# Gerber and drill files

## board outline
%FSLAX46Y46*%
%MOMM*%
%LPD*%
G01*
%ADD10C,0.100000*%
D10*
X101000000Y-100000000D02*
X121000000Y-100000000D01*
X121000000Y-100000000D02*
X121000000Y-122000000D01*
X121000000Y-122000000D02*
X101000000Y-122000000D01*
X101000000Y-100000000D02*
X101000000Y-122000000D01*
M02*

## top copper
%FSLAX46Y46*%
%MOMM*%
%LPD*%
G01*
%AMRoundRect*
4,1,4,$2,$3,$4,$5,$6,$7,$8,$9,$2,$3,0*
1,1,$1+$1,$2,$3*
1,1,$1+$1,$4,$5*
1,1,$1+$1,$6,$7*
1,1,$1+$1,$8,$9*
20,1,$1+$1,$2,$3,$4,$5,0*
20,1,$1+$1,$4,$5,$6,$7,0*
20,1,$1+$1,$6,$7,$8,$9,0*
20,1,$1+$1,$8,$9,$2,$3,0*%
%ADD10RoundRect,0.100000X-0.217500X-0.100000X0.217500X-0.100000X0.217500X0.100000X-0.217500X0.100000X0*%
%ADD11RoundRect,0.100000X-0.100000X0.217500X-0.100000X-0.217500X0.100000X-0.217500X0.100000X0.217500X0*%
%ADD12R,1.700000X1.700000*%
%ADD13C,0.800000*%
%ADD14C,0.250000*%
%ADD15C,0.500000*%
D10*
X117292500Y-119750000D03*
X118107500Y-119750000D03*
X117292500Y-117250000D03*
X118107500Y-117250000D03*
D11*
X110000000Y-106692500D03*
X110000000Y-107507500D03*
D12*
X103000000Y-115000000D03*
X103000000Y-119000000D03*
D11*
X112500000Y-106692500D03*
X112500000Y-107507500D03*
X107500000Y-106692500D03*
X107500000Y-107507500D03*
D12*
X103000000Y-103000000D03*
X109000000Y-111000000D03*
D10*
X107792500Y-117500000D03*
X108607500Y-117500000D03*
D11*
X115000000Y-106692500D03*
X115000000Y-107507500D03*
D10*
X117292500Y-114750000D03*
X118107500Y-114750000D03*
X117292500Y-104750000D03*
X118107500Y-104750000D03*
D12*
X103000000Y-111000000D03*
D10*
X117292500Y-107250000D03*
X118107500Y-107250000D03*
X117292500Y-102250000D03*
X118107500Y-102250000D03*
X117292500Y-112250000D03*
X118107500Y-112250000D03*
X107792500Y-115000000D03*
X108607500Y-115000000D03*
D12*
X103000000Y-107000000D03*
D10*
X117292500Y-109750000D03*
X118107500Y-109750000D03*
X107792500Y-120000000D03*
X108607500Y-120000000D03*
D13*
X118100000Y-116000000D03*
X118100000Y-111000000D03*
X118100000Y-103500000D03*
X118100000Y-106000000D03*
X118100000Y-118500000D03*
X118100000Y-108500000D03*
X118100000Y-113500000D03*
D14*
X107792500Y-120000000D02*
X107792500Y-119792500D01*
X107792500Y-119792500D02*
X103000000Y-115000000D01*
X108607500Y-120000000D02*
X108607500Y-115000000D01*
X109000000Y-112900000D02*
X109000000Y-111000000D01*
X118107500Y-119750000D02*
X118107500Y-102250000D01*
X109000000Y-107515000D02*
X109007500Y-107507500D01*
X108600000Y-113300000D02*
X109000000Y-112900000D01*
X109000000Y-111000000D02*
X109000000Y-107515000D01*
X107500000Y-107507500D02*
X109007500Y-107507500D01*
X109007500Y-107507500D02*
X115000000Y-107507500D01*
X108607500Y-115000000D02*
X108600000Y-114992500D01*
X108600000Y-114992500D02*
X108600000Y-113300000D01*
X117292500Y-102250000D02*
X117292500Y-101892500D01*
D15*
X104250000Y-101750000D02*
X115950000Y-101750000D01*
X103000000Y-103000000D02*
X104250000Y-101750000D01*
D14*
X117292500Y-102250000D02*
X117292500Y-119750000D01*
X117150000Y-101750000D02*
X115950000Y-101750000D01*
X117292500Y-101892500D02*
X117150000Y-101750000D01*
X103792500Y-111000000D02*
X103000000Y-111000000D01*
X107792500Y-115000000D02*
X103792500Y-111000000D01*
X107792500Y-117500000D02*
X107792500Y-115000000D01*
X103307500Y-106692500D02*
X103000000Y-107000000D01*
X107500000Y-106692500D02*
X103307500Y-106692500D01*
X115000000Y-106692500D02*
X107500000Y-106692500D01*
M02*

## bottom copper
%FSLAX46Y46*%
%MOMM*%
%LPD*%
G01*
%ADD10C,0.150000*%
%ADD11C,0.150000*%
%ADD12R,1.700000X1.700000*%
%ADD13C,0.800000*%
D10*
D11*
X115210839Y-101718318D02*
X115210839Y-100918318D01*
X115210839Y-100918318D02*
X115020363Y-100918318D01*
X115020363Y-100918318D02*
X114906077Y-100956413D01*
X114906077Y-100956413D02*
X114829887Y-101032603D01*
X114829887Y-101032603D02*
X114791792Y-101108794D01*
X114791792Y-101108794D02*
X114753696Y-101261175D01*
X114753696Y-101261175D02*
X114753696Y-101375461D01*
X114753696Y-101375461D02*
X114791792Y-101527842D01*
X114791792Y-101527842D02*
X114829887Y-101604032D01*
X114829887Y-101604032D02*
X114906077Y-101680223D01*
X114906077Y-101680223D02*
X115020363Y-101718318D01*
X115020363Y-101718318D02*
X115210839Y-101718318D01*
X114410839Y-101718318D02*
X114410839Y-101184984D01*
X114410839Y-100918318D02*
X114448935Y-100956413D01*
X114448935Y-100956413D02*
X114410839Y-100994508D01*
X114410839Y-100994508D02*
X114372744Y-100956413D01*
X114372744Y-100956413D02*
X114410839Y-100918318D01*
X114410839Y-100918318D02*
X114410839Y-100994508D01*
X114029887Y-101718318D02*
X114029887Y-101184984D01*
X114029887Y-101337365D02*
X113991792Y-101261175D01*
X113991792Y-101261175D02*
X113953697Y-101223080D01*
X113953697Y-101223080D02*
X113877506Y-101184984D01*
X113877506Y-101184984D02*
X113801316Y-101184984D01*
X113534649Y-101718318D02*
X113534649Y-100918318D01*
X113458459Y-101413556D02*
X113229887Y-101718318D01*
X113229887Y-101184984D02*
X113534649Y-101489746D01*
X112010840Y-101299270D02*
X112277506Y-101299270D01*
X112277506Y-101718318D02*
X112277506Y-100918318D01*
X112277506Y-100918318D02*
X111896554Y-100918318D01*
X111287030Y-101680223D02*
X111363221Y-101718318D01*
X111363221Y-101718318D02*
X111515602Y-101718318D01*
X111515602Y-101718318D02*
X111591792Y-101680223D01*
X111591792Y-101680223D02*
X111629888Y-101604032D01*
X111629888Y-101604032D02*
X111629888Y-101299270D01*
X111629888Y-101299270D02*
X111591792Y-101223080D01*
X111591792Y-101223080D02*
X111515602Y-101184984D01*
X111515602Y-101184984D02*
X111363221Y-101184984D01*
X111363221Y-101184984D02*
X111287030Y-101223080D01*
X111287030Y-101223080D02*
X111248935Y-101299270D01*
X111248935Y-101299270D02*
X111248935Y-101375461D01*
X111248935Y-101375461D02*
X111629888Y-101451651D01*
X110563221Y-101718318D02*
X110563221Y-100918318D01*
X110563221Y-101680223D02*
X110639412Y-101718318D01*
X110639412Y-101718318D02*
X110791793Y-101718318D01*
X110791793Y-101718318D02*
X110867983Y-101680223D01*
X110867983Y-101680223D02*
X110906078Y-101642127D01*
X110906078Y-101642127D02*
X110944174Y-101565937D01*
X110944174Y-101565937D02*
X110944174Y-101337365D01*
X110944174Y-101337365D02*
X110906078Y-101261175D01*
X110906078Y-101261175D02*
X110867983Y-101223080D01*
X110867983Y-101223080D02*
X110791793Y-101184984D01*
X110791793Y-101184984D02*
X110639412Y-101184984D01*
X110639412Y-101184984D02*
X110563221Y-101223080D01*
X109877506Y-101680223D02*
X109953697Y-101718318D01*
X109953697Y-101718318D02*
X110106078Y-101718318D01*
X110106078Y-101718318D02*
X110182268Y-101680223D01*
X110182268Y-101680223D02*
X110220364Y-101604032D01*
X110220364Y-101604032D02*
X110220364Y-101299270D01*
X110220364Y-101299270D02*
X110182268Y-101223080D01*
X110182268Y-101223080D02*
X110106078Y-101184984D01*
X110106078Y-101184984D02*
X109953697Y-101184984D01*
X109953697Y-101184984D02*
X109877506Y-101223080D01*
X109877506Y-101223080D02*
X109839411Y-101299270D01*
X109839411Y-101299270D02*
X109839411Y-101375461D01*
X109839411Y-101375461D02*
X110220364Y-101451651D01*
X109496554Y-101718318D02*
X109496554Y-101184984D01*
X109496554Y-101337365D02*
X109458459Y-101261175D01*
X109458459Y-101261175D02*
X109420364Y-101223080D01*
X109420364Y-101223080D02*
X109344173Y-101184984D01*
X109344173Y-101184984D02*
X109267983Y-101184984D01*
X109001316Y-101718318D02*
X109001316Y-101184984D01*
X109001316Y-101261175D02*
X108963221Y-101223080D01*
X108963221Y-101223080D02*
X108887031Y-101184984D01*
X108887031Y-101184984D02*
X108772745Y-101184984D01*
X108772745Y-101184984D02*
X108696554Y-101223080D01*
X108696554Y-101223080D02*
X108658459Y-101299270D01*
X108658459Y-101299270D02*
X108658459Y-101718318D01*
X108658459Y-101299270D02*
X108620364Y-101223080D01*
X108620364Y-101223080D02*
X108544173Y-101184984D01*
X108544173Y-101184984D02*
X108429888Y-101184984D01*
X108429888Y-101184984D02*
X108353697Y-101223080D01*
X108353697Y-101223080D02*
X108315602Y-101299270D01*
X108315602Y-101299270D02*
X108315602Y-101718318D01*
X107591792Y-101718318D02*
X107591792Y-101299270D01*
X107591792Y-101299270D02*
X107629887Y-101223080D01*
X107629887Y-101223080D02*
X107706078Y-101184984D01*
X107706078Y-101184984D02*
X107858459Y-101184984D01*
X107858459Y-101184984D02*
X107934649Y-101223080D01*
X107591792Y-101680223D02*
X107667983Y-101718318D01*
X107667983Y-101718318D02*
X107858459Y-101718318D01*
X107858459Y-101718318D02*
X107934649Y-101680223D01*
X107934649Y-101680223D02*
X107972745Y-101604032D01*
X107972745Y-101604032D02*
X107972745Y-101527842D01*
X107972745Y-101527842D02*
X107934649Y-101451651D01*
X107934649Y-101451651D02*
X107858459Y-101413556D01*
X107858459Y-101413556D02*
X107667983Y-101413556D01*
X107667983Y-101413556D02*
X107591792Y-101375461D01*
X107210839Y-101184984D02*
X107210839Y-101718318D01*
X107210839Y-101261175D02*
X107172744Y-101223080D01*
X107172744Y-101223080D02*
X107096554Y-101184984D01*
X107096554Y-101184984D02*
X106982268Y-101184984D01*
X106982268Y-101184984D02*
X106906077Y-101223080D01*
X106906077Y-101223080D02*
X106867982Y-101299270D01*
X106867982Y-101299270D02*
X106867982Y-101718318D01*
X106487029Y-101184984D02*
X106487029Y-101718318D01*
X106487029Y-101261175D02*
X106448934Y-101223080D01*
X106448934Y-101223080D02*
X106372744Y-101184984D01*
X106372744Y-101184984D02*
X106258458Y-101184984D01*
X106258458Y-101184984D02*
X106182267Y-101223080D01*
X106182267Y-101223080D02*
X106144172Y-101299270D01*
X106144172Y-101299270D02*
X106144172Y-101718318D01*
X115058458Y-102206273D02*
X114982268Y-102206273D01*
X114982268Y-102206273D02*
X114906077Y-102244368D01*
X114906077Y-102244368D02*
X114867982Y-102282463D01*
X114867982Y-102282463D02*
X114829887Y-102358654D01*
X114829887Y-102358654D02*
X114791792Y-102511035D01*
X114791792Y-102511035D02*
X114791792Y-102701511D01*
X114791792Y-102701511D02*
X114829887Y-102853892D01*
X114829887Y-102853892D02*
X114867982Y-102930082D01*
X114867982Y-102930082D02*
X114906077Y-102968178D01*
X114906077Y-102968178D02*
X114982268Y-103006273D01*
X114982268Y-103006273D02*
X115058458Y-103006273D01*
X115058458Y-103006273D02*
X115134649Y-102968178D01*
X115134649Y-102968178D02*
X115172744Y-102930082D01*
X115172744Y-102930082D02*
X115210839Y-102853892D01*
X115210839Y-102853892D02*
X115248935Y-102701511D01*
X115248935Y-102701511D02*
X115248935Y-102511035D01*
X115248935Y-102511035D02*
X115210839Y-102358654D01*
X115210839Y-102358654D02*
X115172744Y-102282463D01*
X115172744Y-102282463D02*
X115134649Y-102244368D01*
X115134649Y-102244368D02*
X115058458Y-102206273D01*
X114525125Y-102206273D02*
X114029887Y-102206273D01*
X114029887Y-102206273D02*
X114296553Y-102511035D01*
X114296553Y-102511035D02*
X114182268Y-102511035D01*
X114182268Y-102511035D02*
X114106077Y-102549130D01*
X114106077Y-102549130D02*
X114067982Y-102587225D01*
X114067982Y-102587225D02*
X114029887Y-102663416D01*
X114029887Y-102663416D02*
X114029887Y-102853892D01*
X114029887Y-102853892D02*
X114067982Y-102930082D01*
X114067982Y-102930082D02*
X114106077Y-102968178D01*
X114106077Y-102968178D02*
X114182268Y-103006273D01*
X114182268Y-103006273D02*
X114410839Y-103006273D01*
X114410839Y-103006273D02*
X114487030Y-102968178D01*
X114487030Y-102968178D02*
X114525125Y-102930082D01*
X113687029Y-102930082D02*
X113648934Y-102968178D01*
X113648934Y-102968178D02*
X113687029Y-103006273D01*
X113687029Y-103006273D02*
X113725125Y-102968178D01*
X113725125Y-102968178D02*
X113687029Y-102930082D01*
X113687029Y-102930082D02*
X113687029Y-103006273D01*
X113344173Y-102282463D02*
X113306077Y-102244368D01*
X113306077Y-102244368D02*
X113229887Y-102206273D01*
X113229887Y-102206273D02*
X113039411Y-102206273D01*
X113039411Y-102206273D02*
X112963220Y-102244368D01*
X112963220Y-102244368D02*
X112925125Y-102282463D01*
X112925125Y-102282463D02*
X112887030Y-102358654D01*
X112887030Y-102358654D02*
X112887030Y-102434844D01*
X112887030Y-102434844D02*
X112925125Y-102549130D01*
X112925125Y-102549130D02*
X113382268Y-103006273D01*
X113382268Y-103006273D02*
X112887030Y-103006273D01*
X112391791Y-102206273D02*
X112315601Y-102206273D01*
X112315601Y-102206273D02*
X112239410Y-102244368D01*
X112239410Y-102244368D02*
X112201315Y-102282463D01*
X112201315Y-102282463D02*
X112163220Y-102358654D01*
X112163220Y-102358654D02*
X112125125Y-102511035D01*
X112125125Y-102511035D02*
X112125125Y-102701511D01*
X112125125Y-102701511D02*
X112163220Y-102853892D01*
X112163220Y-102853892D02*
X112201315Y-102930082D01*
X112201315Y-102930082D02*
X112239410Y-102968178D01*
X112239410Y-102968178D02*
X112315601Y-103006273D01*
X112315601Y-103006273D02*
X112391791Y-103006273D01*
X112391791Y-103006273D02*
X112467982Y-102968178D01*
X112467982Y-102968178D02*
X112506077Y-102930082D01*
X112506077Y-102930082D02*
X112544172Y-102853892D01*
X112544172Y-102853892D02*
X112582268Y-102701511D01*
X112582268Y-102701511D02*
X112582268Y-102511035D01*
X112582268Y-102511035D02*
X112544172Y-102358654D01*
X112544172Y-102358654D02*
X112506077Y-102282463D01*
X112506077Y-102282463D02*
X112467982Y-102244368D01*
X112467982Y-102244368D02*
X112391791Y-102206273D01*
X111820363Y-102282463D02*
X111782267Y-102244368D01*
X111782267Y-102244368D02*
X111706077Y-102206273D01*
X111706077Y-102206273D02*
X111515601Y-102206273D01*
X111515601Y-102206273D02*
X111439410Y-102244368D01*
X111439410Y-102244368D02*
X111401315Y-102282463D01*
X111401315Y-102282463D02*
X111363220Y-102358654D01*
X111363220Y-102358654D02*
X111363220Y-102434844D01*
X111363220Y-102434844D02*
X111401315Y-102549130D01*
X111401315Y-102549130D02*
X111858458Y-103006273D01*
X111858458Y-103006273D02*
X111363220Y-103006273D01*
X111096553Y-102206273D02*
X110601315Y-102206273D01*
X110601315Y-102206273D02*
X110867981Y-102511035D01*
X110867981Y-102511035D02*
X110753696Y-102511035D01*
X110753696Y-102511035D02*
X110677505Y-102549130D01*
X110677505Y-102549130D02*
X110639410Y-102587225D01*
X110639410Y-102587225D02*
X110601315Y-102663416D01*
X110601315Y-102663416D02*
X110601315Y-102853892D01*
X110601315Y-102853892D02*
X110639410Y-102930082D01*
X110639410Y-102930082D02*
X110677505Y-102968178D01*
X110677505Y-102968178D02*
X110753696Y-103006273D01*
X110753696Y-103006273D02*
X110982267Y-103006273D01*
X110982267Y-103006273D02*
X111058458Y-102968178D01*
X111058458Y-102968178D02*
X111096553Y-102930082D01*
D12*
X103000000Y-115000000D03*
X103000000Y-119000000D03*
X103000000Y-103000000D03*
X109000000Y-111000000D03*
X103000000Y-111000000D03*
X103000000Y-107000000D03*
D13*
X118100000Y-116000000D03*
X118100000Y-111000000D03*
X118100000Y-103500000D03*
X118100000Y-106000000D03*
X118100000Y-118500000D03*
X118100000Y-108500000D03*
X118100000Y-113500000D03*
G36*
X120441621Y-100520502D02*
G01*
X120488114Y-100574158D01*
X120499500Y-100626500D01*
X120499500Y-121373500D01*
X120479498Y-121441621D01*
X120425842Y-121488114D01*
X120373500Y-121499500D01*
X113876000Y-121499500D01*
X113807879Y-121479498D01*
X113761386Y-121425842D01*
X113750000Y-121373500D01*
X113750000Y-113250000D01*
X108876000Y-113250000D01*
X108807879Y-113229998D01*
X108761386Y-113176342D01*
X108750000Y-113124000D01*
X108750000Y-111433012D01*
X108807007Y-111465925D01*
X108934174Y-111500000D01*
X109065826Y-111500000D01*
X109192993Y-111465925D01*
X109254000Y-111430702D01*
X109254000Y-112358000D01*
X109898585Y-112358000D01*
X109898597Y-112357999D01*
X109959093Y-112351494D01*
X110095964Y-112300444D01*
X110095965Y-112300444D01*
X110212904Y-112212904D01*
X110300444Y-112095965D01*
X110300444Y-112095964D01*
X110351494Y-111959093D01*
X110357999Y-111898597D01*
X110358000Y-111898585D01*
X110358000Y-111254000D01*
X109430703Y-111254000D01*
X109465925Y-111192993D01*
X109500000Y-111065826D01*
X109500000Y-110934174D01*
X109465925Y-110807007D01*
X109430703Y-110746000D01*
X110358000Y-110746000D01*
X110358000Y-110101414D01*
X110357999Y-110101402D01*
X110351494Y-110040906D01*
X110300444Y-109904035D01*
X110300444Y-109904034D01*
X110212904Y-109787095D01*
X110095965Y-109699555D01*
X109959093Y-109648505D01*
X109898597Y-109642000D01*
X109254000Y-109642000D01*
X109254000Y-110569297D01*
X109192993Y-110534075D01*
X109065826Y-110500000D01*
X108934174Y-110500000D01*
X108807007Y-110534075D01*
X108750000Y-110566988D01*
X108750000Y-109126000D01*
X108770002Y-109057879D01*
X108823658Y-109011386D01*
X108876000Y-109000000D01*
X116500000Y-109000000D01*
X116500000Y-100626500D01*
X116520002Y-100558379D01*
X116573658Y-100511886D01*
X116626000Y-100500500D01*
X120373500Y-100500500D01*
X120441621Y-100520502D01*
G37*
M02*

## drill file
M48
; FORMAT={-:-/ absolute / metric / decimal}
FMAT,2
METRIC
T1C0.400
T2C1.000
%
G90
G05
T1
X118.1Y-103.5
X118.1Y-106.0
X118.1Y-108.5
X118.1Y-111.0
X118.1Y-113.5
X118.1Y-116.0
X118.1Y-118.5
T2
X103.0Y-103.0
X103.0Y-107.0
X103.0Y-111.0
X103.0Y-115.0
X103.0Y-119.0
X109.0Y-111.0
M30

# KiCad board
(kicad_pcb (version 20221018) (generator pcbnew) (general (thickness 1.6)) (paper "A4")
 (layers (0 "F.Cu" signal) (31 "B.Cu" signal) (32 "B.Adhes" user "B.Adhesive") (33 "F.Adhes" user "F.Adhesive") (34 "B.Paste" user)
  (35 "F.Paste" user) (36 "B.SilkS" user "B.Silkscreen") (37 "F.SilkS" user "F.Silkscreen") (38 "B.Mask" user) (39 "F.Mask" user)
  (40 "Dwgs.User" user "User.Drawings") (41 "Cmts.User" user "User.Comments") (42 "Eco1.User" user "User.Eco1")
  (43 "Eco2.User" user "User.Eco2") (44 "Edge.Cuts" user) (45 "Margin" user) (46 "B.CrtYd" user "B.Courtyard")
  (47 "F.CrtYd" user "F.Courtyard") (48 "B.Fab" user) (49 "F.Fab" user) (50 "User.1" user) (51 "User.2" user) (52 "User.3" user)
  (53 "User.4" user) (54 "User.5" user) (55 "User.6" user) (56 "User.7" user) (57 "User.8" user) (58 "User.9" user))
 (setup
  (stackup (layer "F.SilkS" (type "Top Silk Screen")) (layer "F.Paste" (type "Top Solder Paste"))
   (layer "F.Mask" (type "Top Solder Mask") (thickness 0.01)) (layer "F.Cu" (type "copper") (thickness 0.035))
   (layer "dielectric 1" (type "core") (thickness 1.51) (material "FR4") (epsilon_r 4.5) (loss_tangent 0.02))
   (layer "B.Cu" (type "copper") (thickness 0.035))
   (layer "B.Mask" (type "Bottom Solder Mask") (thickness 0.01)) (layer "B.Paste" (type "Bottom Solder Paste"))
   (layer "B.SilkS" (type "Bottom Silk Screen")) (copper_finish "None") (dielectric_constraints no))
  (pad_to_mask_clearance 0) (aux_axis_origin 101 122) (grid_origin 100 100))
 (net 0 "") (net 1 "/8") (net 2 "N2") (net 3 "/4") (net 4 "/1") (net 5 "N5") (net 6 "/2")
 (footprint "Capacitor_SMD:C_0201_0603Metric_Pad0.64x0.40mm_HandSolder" (layer "F.Cu") (at 117.7 119.75)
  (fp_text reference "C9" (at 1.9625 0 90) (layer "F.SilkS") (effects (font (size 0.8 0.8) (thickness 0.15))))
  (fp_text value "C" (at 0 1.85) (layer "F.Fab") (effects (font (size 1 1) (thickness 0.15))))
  (pad "" smd roundrect (at -0.4325 0) (size 0.458 0.36) (layers "F.Paste") (roundrect_rratio 0.25))
  (pad "" smd roundrect (at 0.4325 0) (size 0.458 0.36) (layers "F.Paste") (roundrect_rratio 0.25))
  (pad "1" smd roundrect (at -0.4075 0) (size 0.635 0.4) (layers "F.Cu" "F.Mask") (roundrect_rratio 0.25) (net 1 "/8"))
  (pad "2" smd roundrect (at 0.4075 0) (size 0.635 0.4) (layers "F.Cu" "F.Mask") (roundrect_rratio 0.25) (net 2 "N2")))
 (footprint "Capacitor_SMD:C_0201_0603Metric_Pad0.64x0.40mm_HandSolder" (layer "F.Cu") (at 117.7 117.25)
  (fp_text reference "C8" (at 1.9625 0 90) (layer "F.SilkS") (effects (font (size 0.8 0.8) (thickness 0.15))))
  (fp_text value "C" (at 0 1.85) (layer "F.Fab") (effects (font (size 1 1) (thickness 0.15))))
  (pad "" smd roundrect (at -0.4325 0) (size 0.458 0.36) (layers "F.Paste") (roundrect_rratio 0.25))
  (pad "" smd roundrect (at 0.4325 0) (size 0.458 0.36) (layers "F.Paste") (roundrect_rratio 0.25))
  (pad "1" smd roundrect (at -0.4075 0) (size 0.635 0.4) (layers "F.Cu" "F.Mask") (roundrect_rratio 0.25) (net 1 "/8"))
  (pad "2" smd roundrect (at 0.4075 0) (size 0.635 0.4) (layers "F.Cu" "F.Mask") (roundrect_rratio 0.25) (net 2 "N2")))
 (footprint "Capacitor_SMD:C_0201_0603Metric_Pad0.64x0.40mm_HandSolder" (layer "F.Cu") (at 110 107.1 -90)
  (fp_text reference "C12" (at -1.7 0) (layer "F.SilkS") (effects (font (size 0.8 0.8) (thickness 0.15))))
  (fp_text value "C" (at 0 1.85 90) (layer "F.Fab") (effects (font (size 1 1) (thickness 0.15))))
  (pad "" smd roundrect (at -0.4325 0 270) (size 0.458 0.36) (layers "F.Paste") (roundrect_rratio 0.25))
  (pad "" smd roundrect (at 0.4325 0 270) (size 0.458 0.36) (layers "F.Paste") (roundrect_rratio 0.25))
  (pad "1" smd roundrect (at -0.4075 0 270) (size 0.635 0.4) (layers "F.Cu" "F.Mask") (roundrect_rratio 0.25) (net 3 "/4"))
  (pad "2" smd roundrect (at 0.4075 0 270) (size 0.635 0.4) (layers "F.Cu" "F.Mask") (roundrect_rratio 0.25) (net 2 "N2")))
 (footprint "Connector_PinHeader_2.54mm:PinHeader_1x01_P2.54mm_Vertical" (layer "F.Cu") (at 103 115)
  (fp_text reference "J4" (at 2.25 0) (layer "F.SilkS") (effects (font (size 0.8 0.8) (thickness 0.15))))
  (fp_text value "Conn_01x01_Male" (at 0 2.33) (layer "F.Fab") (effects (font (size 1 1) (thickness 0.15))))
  (pad "1" thru_hole rect (at 0 0) (size 1.7 1.7) (drill 1) (layers "*.Cu" "*.Mask") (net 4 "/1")))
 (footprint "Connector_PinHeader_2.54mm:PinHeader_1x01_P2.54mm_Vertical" (layer "F.Cu") (at 103 119)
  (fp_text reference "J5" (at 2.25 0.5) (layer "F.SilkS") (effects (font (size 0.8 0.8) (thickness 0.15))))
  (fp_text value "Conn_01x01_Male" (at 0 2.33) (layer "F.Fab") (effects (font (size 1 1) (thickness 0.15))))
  (pad "1" thru_hole rect (at 0 0) (size 1.7 1.7) (drill 1) (layers "*.Cu" "*.Mask") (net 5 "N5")))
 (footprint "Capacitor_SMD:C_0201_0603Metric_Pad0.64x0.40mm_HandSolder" (layer "F.Cu") (at 112.5 107.1 -90)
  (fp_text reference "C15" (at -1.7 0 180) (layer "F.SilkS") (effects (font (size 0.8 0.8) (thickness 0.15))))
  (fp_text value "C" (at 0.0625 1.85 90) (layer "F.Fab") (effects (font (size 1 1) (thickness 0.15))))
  (pad "" smd roundrect (at -0.4325 0 270) (size 0.458 0.36) (layers "F.Paste") (roundrect_rratio 0.25))
  (pad "" smd roundrect (at 0.4325 0 270) (size 0.458 0.36) (layers "F.Paste") (roundrect_rratio 0.25))
  (pad "1" smd roundrect (at -0.4075 0 270) (size 0.635 0.4) (layers "F.Cu" "F.Mask") (roundrect_rratio 0.25) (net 3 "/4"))
  (pad "2" smd roundrect (at 0.4075 0 270) (size 0.635 0.4) (layers "F.Cu" "F.Mask") (roundrect_rratio 0.25) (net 2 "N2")))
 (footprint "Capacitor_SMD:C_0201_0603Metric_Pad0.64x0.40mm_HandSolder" (layer "F.Cu") (at 107.5 107.1 -90)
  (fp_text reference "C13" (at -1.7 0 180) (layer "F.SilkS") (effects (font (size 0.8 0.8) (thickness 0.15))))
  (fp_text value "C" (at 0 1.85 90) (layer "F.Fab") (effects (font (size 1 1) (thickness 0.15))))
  (pad "" smd roundrect (at -0.4325 0 270) (size 0.458 0.36) (layers "F.Paste") (roundrect_rratio 0.25))
  (pad "" smd roundrect (at 0.4325 0 270) (size 0.458 0.36) (layers "F.Paste") (roundrect_rratio 0.25))
  (pad "1" smd roundrect (at -0.4075 0 270) (size 0.635 0.4) (layers "F.Cu" "F.Mask") (roundrect_rratio 0.25) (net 3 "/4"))
  (pad "2" smd roundrect (at 0.4075 0 270) (size 0.635 0.4) (layers "F.Cu" "F.Mask") (roundrect_rratio 0.25) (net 2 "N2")))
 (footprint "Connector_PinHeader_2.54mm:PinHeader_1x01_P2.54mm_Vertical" (layer "F.Cu") (at 103 103)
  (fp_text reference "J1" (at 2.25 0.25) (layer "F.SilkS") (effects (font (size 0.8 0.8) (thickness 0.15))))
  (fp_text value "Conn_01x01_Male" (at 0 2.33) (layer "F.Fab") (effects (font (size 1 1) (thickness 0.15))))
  (pad "1" thru_hole rect (at 0 0) (size 1.7 1.7) (drill 1) (layers "*.Cu" "*.Mask") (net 1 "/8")))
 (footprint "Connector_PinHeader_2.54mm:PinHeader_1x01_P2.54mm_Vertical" (layer "F.Cu") (at 109 111)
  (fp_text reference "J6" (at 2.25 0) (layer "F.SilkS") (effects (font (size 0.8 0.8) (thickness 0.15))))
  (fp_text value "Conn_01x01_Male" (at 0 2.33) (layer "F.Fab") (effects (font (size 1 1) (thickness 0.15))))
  (pad "1" thru_hole rect (at 0 0) (size 1.7 1.7) (drill 1) (layers "*.Cu" "*.Mask") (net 2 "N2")))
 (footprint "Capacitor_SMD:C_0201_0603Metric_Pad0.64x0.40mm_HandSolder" (layer "F.Cu") (at 108.2 117.5)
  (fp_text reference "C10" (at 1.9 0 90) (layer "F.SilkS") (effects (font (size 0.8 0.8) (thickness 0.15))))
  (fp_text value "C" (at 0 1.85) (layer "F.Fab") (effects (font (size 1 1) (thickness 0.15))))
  (pad "" smd roundrect (at -0.4325 0) (size 0.458 0.36) (layers "F.Paste") (roundrect_rratio 0.25))
  (pad "" smd roundrect (at 0.4325 0) (size 0.458 0.36) (layers "F.Paste") (roundrect_rratio 0.25))
  (pad "1" smd roundrect (at -0.4075 0) (size 0.635 0.4) (layers "F.Cu" "F.Mask") (roundrect_rratio 0.25) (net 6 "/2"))
  (pad "2" smd roundrect (at 0.4075 0) (size 0.635 0.4) (layers "F.Cu" "F.Mask") (roundrect_rratio 0.25) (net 2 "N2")))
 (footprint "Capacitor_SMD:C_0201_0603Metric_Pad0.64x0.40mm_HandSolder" (layer "F.Cu") (at 115 107.1 -90)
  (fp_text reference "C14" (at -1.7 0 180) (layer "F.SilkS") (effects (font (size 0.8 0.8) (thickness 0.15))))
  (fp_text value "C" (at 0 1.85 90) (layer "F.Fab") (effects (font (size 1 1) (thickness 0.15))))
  (pad "" smd roundrect (at -0.4325 0 270) (size 0.458 0.36) (layers "F.Paste") (roundrect_rratio 0.25))
  (pad "" smd roundrect (at 0.4325 0 270) (size 0.458 0.36) (layers "F.Paste") (roundrect_rratio 0.25))
  (pad "1" smd roundrect (at -0.4075 0 270) (size 0.635 0.4) (layers "F.Cu" "F.Mask") (roundrect_rratio 0.25) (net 3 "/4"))
  (pad "2" smd roundrect (at 0.4075 0 270) (size 0.635 0.4) (layers "F.Cu" "F.Mask") (roundrect_rratio 0.25) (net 2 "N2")))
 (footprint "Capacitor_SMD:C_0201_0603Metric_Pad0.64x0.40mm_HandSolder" (layer "F.Cu") (at 117.7 114.75)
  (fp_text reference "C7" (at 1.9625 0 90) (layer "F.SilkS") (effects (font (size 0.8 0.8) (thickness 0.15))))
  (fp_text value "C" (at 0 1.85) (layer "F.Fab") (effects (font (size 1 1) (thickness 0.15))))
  (pad "" smd roundrect (at -0.4325 0) (size 0.458 0.36) (layers "F.Paste") (roundrect_rratio 0.25))
  (pad "" smd roundrect (at 0.4325 0) (size 0.458 0.36) (layers "F.Paste") (roundrect_rratio 0.25))
  (pad "1" smd roundrect (at -0.4075 0) (size 0.635 0.4) (layers "F.Cu" "F.Mask") (roundrect_rratio 0.25) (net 1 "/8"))
  (pad "2" smd roundrect (at 0.4075 0) (size 0.635 0.4) (layers "F.Cu" "F.Mask") (roundrect_rratio 0.25) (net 2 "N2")))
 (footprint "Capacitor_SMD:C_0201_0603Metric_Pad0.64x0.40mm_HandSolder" (layer "F.Cu") (at 117.7 104.75)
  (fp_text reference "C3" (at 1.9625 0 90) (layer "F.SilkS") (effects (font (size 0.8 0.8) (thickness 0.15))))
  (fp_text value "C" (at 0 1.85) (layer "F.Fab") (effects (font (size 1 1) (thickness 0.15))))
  (pad "" smd roundrect (at -0.4325 0) (size 0.458 0.36) (layers "F.Paste") (roundrect_rratio 0.25))
  (pad "" smd roundrect (at 0.4325 0) (size 0.458 0.36) (layers "F.Paste") (roundrect_rratio 0.25))
  (pad "1" smd roundrect (at -0.4075 0) (size 0.635 0.4) (layers "F.Cu" "F.Mask") (roundrect_rratio 0.25) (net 1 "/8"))
  (pad "2" smd roundrect (at 0.4075 0) (size 0.635 0.4) (layers "F.Cu" "F.Mask") (roundrect_rratio 0.25) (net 2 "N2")))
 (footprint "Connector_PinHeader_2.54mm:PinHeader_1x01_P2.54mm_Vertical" (layer "F.Cu") (at 103 111)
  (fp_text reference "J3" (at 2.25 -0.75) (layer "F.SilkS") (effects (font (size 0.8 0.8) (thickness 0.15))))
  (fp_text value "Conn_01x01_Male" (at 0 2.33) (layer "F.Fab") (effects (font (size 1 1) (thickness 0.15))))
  (pad "1" thru_hole rect (at 0 0) (size 1.7 1.7) (drill 1) (layers "*.Cu" "*.Mask") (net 6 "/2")))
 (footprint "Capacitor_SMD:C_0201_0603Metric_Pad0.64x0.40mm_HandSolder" (layer "F.Cu") (at 117.7 107.25)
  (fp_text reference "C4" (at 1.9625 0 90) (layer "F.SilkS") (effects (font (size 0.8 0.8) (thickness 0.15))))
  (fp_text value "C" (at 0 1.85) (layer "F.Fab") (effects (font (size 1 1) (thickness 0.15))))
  (pad "" smd roundrect (at -0.4325 0) (size 0.458 0.36) (layers "F.Paste") (roundrect_rratio 0.25))
  (pad "" smd roundrect (at 0.4325 0) (size 0.458 0.36) (layers "F.Paste") (roundrect_rratio 0.25))
  (pad "1" smd roundrect (at -0.4075 0) (size 0.635 0.4) (layers "F.Cu" "F.Mask") (roundrect_rratio 0.25) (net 1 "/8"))
  (pad "2" smd roundrect (at 0.4075 0) (size 0.635 0.4) (layers "F.Cu" "F.Mask") (roundrect_rratio 0.25) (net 2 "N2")))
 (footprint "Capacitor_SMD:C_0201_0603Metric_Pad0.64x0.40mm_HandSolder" (layer "F.Cu") (at 117.7 102.25)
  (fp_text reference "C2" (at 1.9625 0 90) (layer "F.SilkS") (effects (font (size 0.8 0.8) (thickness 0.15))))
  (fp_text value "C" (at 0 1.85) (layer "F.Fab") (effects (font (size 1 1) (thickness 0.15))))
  (pad "" smd roundrect (at -0.4325 0) (size 0.458 0.36) (layers "F.Paste") (roundrect_rratio 0.25))
  (pad "" smd roundrect (at 0.4325 0) (size 0.458 0.36) (layers "F.Paste") (roundrect_rratio 0.25))
  (pad "1" smd roundrect (at -0.4075 0) (size 0.635 0.4) (layers "F.Cu" "F.Mask") (roundrect_rratio 0.25) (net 1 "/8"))
  (pad "2" smd roundrect (at 0.4075 0) (size 0.635 0.4) (layers "F.Cu" "F.Mask") (roundrect_rratio 0.25) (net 2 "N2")))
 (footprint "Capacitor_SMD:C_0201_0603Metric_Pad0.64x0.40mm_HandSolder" (layer "F.Cu") (at 117.7 112.25)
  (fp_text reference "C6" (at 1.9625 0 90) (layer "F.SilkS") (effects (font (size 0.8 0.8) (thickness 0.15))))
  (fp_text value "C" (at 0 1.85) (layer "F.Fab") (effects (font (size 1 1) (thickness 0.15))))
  (pad "" smd roundrect (at -0.4325 0) (size 0.458 0.36) (layers "F.Paste") (roundrect_rratio 0.25))
  (pad "" smd roundrect (at 0.4325 0) (size 0.458 0.36) (layers "F.Paste") (roundrect_rratio 0.25))
  (pad "1" smd roundrect (at -0.4075 0) (size 0.635 0.4) (layers "F.Cu" "F.Mask") (roundrect_rratio 0.25) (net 1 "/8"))
  (pad "2" smd roundrect (at 0.4075 0) (size 0.635 0.4) (layers "F.Cu" "F.Mask") (roundrect_rratio 0.25) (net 2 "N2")))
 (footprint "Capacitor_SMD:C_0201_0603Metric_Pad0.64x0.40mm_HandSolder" (layer "F.Cu") (at 108.2 115)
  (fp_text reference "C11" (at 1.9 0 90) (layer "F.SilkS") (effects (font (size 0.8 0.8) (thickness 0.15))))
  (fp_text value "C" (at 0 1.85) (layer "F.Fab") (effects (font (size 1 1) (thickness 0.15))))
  (pad "" smd roundrect (at -0.4325 0) (size 0.458 0.36) (layers "F.Paste") (roundrect_rratio 0.25))
  (pad "" smd roundrect (at 0.4325 0) (size 0.458 0.36) (layers "F.Paste") (roundrect_rratio 0.25))
  (pad "1" smd roundrect (at -0.4075 0) (size 0.635 0.4) (layers "F.Cu" "F.Mask") (roundrect_rratio 0.25) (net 6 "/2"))
  (pad "2" smd roundrect (at 0.4075 0) (size 0.635 0.4) (layers "F.Cu" "F.Mask") (roundrect_rratio 0.25) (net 2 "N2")))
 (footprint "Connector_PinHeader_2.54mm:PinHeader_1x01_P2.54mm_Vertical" (layer "F.Cu") (at 103 107)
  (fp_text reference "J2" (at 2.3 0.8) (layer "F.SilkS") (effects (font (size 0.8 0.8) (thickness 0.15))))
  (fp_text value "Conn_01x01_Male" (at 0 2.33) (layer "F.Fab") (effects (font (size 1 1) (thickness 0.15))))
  (pad "1" thru_hole rect (at 0 0) (size 1.7 1.7) (drill 1) (layers "*.Cu" "*.Mask") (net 3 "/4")))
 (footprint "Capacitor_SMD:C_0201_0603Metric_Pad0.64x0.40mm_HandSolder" (layer "F.Cu") (at 117.7 109.75)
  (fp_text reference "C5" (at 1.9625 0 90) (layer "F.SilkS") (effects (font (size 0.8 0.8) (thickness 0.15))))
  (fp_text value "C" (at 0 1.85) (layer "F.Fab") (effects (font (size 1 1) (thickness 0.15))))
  (pad "" smd roundrect (at -0.4325 0) (size 0.458 0.36) (layers "F.Paste") (roundrect_rratio 0.25))
  (pad "" smd roundrect (at 0.4325 0) (size 0.458 0.36) (layers "F.Paste") (roundrect_rratio 0.25))
  (pad "1" smd roundrect (at -0.4075 0) (size 0.635 0.4) (layers "F.Cu" "F.Mask") (roundrect_rratio 0.25) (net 1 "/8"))
  (pad "2" smd roundrect (at 0.4075 0) (size 0.635 0.4) (layers "F.Cu" "F.Mask") (roundrect_rratio 0.25) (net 2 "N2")))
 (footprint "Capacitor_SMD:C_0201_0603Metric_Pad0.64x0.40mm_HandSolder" (layer "F.Cu") (at 108.2 120)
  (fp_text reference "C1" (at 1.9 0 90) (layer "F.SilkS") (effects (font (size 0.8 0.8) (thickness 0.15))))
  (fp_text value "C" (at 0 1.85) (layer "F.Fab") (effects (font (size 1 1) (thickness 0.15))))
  (pad "" smd roundrect (at -0.4325 0) (size 0.458 0.36) (layers "F.Paste") (roundrect_rratio 0.25))
  (pad "" smd roundrect (at 0.4325 0) (size 0.458 0.36) (layers "F.Paste") (roundrect_rratio 0.25))
  (pad "1" smd roundrect (at -0.4075 0) (size 0.635 0.4) (layers "F.Cu" "F.Mask") (roundrect_rratio 0.25) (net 4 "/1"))
  (pad "2" smd roundrect (at 0.4075 0) (size 0.635 0.4) (layers "F.Cu" "F.Mask") (roundrect_rratio 0.25) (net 2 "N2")))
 (gr_line (start 101 100) (end 121 100) (stroke (width 0.1) (type solid)) (layer "Edge.Cuts"))
 (gr_line (start 121 100) (end 121 122) (stroke (width 0.1) (type solid)) (layer "Edge.Cuts"))
 (gr_line (start 121 122) (end 101 122) (stroke (width 0.1) (type solid)) (layer "Edge.Cuts"))
 (gr_line (start 101 100) (end 101 122) (stroke (width 0.1) (type solid)) (layer "Edge.Cuts"))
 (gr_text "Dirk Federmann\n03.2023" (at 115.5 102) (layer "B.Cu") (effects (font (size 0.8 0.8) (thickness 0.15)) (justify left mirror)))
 (segment (start 107.7925 120) (end 107.7925 119.7925) (width 0.25) (layer "F.Cu") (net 4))
 (segment (start 107.7925 119.7925) (end 103 115) (width 0.25) (layer "F.Cu") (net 4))
 (segment (start 108.6075 120) (end 108.6075 115) (width 0.25) (layer "F.Cu") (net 2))
 (segment (start 109 112.9) (end 109 111) (width 0.25) (layer "F.Cu") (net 2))
 (segment (start 118.1075 119.75) (end 118.1075 102.25) (width 0.25) (layer "F.Cu") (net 2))
 (segment (start 109 107.515) (end 109.0075 107.5075) (width 0.25) (layer "F.Cu") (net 2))
 (segment (start 108.6 113.3) (end 109 112.9) (width 0.25) (layer "F.Cu") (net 2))
 (segment (start 109 111) (end 109 107.515) (width 0.25) (layer "F.Cu") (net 2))
 (segment (start 107.5 107.5075) (end 109.0075 107.5075) (width 0.25) (layer "F.Cu") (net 2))
 (segment (start 109.0075 107.5075) (end 115 107.5075) (width 0.25) (layer "F.Cu") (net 2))
 (segment (start 108.6075 115) (end 108.6 114.9925) (width 0.25) (layer "F.Cu") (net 2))
 (segment (start 108.6 114.9925) (end 108.6 113.3) (width 0.25) (layer "F.Cu") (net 2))
 (via (at 118.1 116) (size 0.8) (drill 0.4) (layers "F.Cu" "B.Cu") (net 2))
 (via (at 118.1 111) (size 0.8) (drill 0.4) (layers "F.Cu" "B.Cu") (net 2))
 (via (at 118.1 103.5) (size 0.8) (drill 0.4) (layers "F.Cu" "B.Cu") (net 2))
 (via (at 118.1 106) (size 0.8) (drill 0.4) (layers "F.Cu" "B.Cu") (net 2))
 (via (at 118.1 118.5) (size 0.8) (drill 0.4) (layers "F.Cu" "B.Cu") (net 2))
 (via (at 118.1 108.5) (size 0.8) (drill 0.4) (layers "F.Cu" "B.Cu") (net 2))
 (via (at 118.1 113.5) (size 0.8) (drill 0.4) (layers "F.Cu" "B.Cu") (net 2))
 (segment (start 117.2925 102.25) (end 117.2925 101.8925) (width 0.25) (layer "F.Cu") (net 1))
 (segment (start 104.25 101.75) (end 115.95 101.75) (width 0.5) (layer "F.Cu") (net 1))
 (segment (start 103 103) (end 104.25 101.75) (width 0.5) (layer "F.Cu") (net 1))
 (segment (start 117.2925 102.25) (end 117.2925 119.75) (width 0.25) (layer "F.Cu") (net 1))
 (segment (start 117.15 101.75) (end 115.95 101.75) (width 0.25) (layer "F.Cu") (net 1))
 (segment (start 117.2925 101.8925) (end 117.15 101.75) (width 0.25) (layer "F.Cu") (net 1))
 (segment (start 103.7925 111) (end 103 111) (width 0.25) (layer "F.Cu") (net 6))
 (segment (start 107.7925 115) (end 103.7925 111) (width 0.25) (layer "F.Cu") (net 6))
 (segment (start 107.7925 117.5) (end 107.7925 115) (width 0.25) (layer "F.Cu") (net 6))
 (segment (start 103.3075 106.6925) (end 103 107) (width 0.25) (layer "F.Cu") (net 3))
 (segment (start 107.5 106.6925) (end 103.3075 106.6925) (width 0.25) (layer "F.Cu") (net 3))
 (segment (start 115 106.6925) (end 107.5 106.6925) (width 0.25) (layer "F.Cu") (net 3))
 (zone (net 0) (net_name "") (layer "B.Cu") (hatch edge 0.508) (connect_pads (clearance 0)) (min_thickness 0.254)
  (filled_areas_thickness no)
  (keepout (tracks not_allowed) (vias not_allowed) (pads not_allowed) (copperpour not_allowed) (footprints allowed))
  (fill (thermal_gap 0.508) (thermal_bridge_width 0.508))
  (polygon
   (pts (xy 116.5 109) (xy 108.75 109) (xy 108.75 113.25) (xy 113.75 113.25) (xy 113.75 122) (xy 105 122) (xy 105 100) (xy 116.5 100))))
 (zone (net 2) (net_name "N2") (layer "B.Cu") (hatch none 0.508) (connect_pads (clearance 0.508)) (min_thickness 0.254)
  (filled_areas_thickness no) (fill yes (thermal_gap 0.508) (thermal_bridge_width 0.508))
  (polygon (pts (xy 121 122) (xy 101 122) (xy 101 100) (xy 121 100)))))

